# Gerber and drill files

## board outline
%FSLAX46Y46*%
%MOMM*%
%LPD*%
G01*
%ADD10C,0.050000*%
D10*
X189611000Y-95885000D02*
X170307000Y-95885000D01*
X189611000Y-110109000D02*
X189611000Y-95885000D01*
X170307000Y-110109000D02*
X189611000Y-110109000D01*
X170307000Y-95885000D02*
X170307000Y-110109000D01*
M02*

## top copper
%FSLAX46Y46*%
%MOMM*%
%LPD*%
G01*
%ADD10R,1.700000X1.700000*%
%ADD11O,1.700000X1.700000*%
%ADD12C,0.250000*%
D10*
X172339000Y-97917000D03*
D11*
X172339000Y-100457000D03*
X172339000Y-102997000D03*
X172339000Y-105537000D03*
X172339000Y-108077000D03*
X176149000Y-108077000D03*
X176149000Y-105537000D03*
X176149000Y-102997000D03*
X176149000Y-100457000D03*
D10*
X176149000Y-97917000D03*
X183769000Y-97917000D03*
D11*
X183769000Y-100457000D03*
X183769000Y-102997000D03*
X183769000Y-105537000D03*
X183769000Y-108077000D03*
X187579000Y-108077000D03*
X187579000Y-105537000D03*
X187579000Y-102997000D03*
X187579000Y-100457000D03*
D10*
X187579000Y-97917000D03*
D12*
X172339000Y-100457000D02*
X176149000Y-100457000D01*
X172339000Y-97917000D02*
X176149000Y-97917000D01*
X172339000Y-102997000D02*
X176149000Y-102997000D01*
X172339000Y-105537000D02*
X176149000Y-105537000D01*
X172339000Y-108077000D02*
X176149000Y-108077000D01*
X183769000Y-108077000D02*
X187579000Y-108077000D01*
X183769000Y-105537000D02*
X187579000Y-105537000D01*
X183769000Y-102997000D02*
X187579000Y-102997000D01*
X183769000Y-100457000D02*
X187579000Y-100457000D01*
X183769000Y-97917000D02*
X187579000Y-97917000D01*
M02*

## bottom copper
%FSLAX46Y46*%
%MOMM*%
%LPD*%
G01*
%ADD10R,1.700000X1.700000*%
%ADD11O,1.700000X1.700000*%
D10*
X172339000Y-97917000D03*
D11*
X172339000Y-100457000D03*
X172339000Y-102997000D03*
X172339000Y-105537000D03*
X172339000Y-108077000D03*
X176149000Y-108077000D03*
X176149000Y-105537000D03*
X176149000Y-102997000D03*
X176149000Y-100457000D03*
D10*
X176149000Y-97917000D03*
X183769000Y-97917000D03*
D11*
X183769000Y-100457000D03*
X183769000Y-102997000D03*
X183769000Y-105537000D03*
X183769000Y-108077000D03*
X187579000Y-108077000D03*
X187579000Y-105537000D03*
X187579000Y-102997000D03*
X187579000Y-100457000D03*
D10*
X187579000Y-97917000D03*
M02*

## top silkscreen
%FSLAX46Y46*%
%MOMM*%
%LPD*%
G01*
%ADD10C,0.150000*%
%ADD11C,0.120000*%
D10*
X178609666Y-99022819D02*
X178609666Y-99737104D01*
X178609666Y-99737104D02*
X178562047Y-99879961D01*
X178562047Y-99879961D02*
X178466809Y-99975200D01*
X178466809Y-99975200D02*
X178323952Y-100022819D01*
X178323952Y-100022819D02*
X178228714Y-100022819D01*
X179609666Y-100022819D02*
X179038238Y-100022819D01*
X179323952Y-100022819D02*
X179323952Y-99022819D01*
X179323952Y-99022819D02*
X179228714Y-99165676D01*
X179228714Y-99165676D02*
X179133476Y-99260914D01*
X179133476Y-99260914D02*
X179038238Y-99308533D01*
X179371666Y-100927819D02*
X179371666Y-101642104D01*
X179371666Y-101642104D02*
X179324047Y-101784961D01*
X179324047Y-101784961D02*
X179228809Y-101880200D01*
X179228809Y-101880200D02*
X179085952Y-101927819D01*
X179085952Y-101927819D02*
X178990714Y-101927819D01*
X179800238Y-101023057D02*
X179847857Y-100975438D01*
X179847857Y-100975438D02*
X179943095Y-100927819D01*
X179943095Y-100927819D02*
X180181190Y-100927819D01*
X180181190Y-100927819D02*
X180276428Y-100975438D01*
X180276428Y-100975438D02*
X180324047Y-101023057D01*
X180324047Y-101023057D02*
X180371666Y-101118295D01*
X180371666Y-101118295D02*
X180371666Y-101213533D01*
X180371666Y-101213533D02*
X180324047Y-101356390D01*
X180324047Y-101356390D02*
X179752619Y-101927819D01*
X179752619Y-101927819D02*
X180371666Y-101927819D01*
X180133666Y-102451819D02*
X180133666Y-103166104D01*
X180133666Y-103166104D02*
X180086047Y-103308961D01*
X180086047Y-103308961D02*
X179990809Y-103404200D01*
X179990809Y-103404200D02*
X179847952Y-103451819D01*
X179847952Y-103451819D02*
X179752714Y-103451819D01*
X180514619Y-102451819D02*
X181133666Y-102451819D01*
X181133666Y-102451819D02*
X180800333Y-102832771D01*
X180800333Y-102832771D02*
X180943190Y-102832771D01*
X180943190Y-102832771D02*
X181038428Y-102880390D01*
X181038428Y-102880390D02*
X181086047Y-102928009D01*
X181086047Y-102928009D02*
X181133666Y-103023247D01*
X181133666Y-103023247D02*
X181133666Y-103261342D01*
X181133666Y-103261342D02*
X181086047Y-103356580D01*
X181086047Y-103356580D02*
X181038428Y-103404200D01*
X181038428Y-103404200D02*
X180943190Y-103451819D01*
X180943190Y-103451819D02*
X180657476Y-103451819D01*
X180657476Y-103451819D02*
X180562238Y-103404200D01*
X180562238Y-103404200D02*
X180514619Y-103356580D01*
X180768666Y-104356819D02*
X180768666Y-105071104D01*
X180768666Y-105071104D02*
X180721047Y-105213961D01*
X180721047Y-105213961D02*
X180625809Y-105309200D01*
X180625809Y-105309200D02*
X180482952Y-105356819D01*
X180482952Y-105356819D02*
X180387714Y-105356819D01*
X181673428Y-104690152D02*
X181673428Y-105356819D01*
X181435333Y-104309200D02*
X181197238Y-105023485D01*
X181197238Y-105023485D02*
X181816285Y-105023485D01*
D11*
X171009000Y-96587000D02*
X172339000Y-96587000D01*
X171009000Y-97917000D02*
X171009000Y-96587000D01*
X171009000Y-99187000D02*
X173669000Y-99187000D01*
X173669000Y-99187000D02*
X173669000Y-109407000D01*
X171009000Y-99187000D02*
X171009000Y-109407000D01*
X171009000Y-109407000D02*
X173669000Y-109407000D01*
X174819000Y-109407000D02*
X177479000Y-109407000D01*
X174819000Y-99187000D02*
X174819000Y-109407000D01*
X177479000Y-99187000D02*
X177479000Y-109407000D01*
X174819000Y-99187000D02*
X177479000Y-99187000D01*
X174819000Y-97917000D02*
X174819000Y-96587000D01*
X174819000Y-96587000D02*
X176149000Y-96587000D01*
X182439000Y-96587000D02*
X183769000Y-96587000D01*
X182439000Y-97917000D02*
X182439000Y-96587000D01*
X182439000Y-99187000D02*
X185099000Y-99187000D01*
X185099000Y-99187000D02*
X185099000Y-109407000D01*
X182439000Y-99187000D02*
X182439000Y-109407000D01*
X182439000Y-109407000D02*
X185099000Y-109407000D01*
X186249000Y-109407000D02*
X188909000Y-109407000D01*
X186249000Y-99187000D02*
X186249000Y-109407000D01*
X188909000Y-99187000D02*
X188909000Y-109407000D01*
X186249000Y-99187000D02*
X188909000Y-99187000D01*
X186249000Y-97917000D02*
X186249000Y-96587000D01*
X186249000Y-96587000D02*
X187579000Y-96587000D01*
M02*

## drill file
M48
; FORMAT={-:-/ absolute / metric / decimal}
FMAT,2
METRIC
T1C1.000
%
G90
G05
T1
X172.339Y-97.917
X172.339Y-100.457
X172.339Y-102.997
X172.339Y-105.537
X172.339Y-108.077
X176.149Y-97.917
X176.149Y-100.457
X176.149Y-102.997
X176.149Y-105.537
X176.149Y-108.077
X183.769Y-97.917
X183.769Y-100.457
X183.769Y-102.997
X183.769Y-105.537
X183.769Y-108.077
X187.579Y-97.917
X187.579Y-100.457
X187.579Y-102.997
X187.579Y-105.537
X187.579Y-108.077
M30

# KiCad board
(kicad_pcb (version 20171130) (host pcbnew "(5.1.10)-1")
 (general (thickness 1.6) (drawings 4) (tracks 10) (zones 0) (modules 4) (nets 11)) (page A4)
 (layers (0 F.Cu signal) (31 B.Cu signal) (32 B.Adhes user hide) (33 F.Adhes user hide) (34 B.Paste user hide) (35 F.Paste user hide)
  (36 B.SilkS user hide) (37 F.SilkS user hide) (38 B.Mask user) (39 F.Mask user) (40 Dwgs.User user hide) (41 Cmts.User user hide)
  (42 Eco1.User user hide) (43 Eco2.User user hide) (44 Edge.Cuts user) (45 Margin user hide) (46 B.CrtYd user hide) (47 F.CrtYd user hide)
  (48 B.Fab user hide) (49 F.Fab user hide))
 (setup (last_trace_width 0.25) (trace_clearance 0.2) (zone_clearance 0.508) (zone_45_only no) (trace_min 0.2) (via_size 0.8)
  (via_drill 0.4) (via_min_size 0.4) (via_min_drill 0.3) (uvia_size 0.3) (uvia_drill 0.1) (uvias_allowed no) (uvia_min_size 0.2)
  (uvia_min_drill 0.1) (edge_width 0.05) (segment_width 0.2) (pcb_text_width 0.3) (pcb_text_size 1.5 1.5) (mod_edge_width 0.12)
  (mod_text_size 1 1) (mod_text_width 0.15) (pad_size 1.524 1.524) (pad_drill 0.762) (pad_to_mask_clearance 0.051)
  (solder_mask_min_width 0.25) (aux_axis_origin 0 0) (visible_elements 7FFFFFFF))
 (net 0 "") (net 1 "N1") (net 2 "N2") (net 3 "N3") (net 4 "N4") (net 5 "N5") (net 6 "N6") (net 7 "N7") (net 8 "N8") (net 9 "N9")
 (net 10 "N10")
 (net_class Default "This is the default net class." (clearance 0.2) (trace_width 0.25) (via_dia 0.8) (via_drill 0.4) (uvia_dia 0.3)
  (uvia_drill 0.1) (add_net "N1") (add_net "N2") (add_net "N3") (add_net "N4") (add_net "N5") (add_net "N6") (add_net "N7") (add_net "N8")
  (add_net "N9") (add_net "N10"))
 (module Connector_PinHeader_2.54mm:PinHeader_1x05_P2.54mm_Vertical (layer F.Cu) (at 172.339 97.917)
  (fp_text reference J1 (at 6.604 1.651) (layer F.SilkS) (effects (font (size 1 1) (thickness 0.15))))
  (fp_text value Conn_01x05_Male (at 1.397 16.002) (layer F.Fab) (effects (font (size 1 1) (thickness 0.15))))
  (fp_line (start -1.33 -1.33) (end 0 -1.33) (layer F.SilkS) (width 0.12))
  (fp_line (start -1.33 0) (end -1.33 -1.33) (layer F.SilkS) (width 0.12))
  (fp_line (start -1.33 1.27) (end 1.33 1.27) (layer F.SilkS) (width 0.12))
  (fp_line (start 1.33 1.27) (end 1.33 11.49) (layer F.SilkS) (width 0.12))
  (fp_line (start -1.33 1.27) (end -1.33 11.49) (layer F.SilkS) (width 0.12))
  (fp_line (start -1.33 11.49) (end 1.33 11.49) (layer F.SilkS) (width 0.12))
  (pad 1 thru_hole rect (at 0 0) (size 1.7 1.7) (drill 1) (layers *.Cu *.Mask) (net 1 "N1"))
  (pad 2 thru_hole oval (at 0 2.54) (size 1.7 1.7) (drill 1) (layers *.Cu *.Mask) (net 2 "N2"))
  (pad 3 thru_hole oval (at 0 5.08) (size 1.7 1.7) (drill 1) (layers *.Cu *.Mask) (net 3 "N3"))
  (pad 4 thru_hole oval (at 0 7.62) (size 1.7 1.7) (drill 1) (layers *.Cu *.Mask) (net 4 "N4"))
  (pad 5 thru_hole oval (at 0 10.16) (size 1.7 1.7) (drill 1) (layers *.Cu *.Mask) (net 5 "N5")))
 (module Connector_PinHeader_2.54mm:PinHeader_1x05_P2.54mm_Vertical (layer F.Cu) (at 176.149 97.917)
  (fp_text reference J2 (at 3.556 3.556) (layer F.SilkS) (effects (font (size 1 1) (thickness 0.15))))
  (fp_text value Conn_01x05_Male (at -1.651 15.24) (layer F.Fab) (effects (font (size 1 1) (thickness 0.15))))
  (fp_line (start -1.33 11.49) (end 1.33 11.49) (layer F.SilkS) (width 0.12))
  (fp_line (start -1.33 1.27) (end -1.33 11.49) (layer F.SilkS) (width 0.12))
  (fp_line (start 1.33 1.27) (end 1.33 11.49) (layer F.SilkS) (width 0.12))
  (fp_line (start -1.33 1.27) (end 1.33 1.27) (layer F.SilkS) (width 0.12))
  (fp_line (start -1.33 0) (end -1.33 -1.33) (layer F.SilkS) (width 0.12))
  (fp_line (start -1.33 -1.33) (end 0 -1.33) (layer F.SilkS) (width 0.12))
  (pad 5 thru_hole oval (at 0 10.16) (size 1.7 1.7) (drill 1) (layers *.Cu *.Mask) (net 5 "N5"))
  (pad 4 thru_hole oval (at 0 7.62) (size 1.7 1.7) (drill 1) (layers *.Cu *.Mask) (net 4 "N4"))
  (pad 3 thru_hole oval (at 0 5.08) (size 1.7 1.7) (drill 1) (layers *.Cu *.Mask) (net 3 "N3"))
  (pad 2 thru_hole oval (at 0 2.54) (size 1.7 1.7) (drill 1) (layers *.Cu *.Mask) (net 2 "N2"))
  (pad 1 thru_hole rect (at 0 0) (size 1.7 1.7) (drill 1) (layers *.Cu *.Mask) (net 1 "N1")))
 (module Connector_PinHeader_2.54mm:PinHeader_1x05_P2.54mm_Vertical (layer F.Cu) (at 183.769 97.917)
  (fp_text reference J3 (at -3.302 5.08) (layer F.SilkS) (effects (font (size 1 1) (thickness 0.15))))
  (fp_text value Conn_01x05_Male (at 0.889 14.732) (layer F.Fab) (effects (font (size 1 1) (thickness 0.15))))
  (fp_line (start -1.33 -1.33) (end 0 -1.33) (layer F.SilkS) (width 0.12))
  (fp_line (start -1.33 0) (end -1.33 -1.33) (layer F.SilkS) (width 0.12))
  (fp_line (start -1.33 1.27) (end 1.33 1.27) (layer F.SilkS) (width 0.12))
  (fp_line (start 1.33 1.27) (end 1.33 11.49) (layer F.SilkS) (width 0.12))
  (fp_line (start -1.33 1.27) (end -1.33 11.49) (layer F.SilkS) (width 0.12))
  (fp_line (start -1.33 11.49) (end 1.33 11.49) (layer F.SilkS) (width 0.12))
  (pad 1 thru_hole rect (at 0 0) (size 1.7 1.7) (drill 1) (layers *.Cu *.Mask) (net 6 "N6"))
  (pad 2 thru_hole oval (at 0 2.54) (size 1.7 1.7) (drill 1) (layers *.Cu *.Mask) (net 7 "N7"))
  (pad 3 thru_hole oval (at 0 5.08) (size 1.7 1.7) (drill 1) (layers *.Cu *.Mask) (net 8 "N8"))
  (pad 4 thru_hole oval (at 0 7.62) (size 1.7 1.7) (drill 1) (layers *.Cu *.Mask) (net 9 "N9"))
  (pad 5 thru_hole oval (at 0 10.16) (size 1.7 1.7) (drill 1) (layers *.Cu *.Mask) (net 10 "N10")))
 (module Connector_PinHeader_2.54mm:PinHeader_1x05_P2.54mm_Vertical (layer F.Cu) (at 187.579 97.917)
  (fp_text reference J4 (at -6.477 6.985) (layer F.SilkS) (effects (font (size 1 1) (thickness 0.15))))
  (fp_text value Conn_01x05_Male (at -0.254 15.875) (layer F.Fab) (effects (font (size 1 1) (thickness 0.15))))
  (fp_line (start -1.33 11.49) (end 1.33 11.49) (layer F.SilkS) (width 0.12))
  (fp_line (start -1.33 1.27) (end -1.33 11.49) (layer F.SilkS) (width 0.12))
  (fp_line (start 1.33 1.27) (end 1.33 11.49) (layer F.SilkS) (width 0.12))
  (fp_line (start -1.33 1.27) (end 1.33 1.27) (layer F.SilkS) (width 0.12))
  (fp_line (start -1.33 0) (end -1.33 -1.33) (layer F.SilkS) (width 0.12))
  (fp_line (start -1.33 -1.33) (end 0 -1.33) (layer F.SilkS) (width 0.12))
  (pad 5 thru_hole oval (at 0 10.16) (size 1.7 1.7) (drill 1) (layers *.Cu *.Mask) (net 10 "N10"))
  (pad 4 thru_hole oval (at 0 7.62) (size 1.7 1.7) (drill 1) (layers *.Cu *.Mask) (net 9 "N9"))
  (pad 3 thru_hole oval (at 0 5.08) (size 1.7 1.7) (drill 1) (layers *.Cu *.Mask) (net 8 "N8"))
  (pad 2 thru_hole oval (at 0 2.54) (size 1.7 1.7) (drill 1) (layers *.Cu *.Mask) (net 7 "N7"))
  (pad 1 thru_hole rect (at 0 0) (size 1.7 1.7) (drill 1) (layers *.Cu *.Mask) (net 6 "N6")))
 (gr_line (start 189.611 95.885) (end 170.307 95.885) (layer Edge.Cuts) (width 0.05))
 (gr_line (start 189.611 110.109) (end 189.611 95.885) (layer Edge.Cuts) (width 0.05))
 (gr_line (start 170.307 110.109) (end 189.611 110.109) (layer Edge.Cuts) (width 0.05))
 (gr_line (start 170.307 95.885) (end 170.307 110.109) (layer Edge.Cuts) (width 0.05))
 (segment (start 172.339 100.457) (end 176.149 100.457) (width 0.25) (layer F.Cu) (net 2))
 (segment (start 172.339 97.917) (end 176.149 97.917) (width 0.25) (layer F.Cu) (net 1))
 (segment (start 172.339 102.997) (end 176.149 102.997) (width 0.25) (layer F.Cu) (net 3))
 (segment (start 172.339 105.537) (end 176.149 105.537) (width 0.25) (layer F.Cu) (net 4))
 (segment (start 172.339 108.077) (end 176.149 108.077) (width 0.25) (layer F.Cu) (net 5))
 (segment (start 183.769 108.077) (end 187.579 108.077) (width 0.25) (layer F.Cu) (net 10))
 (segment (start 183.769 105.537) (end 187.579 105.537) (width 0.25) (layer F.Cu) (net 9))
 (segment (start 183.769 102.997) (end 187.579 102.997) (width 0.25) (layer F.Cu) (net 8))
 (segment (start 183.769 100.457) (end 187.579 100.457) (width 0.25) (layer F.Cu) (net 7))
 (segment (start 183.769 97.917) (end 187.579 97.917) (width 0.25) (layer F.Cu) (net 6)))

